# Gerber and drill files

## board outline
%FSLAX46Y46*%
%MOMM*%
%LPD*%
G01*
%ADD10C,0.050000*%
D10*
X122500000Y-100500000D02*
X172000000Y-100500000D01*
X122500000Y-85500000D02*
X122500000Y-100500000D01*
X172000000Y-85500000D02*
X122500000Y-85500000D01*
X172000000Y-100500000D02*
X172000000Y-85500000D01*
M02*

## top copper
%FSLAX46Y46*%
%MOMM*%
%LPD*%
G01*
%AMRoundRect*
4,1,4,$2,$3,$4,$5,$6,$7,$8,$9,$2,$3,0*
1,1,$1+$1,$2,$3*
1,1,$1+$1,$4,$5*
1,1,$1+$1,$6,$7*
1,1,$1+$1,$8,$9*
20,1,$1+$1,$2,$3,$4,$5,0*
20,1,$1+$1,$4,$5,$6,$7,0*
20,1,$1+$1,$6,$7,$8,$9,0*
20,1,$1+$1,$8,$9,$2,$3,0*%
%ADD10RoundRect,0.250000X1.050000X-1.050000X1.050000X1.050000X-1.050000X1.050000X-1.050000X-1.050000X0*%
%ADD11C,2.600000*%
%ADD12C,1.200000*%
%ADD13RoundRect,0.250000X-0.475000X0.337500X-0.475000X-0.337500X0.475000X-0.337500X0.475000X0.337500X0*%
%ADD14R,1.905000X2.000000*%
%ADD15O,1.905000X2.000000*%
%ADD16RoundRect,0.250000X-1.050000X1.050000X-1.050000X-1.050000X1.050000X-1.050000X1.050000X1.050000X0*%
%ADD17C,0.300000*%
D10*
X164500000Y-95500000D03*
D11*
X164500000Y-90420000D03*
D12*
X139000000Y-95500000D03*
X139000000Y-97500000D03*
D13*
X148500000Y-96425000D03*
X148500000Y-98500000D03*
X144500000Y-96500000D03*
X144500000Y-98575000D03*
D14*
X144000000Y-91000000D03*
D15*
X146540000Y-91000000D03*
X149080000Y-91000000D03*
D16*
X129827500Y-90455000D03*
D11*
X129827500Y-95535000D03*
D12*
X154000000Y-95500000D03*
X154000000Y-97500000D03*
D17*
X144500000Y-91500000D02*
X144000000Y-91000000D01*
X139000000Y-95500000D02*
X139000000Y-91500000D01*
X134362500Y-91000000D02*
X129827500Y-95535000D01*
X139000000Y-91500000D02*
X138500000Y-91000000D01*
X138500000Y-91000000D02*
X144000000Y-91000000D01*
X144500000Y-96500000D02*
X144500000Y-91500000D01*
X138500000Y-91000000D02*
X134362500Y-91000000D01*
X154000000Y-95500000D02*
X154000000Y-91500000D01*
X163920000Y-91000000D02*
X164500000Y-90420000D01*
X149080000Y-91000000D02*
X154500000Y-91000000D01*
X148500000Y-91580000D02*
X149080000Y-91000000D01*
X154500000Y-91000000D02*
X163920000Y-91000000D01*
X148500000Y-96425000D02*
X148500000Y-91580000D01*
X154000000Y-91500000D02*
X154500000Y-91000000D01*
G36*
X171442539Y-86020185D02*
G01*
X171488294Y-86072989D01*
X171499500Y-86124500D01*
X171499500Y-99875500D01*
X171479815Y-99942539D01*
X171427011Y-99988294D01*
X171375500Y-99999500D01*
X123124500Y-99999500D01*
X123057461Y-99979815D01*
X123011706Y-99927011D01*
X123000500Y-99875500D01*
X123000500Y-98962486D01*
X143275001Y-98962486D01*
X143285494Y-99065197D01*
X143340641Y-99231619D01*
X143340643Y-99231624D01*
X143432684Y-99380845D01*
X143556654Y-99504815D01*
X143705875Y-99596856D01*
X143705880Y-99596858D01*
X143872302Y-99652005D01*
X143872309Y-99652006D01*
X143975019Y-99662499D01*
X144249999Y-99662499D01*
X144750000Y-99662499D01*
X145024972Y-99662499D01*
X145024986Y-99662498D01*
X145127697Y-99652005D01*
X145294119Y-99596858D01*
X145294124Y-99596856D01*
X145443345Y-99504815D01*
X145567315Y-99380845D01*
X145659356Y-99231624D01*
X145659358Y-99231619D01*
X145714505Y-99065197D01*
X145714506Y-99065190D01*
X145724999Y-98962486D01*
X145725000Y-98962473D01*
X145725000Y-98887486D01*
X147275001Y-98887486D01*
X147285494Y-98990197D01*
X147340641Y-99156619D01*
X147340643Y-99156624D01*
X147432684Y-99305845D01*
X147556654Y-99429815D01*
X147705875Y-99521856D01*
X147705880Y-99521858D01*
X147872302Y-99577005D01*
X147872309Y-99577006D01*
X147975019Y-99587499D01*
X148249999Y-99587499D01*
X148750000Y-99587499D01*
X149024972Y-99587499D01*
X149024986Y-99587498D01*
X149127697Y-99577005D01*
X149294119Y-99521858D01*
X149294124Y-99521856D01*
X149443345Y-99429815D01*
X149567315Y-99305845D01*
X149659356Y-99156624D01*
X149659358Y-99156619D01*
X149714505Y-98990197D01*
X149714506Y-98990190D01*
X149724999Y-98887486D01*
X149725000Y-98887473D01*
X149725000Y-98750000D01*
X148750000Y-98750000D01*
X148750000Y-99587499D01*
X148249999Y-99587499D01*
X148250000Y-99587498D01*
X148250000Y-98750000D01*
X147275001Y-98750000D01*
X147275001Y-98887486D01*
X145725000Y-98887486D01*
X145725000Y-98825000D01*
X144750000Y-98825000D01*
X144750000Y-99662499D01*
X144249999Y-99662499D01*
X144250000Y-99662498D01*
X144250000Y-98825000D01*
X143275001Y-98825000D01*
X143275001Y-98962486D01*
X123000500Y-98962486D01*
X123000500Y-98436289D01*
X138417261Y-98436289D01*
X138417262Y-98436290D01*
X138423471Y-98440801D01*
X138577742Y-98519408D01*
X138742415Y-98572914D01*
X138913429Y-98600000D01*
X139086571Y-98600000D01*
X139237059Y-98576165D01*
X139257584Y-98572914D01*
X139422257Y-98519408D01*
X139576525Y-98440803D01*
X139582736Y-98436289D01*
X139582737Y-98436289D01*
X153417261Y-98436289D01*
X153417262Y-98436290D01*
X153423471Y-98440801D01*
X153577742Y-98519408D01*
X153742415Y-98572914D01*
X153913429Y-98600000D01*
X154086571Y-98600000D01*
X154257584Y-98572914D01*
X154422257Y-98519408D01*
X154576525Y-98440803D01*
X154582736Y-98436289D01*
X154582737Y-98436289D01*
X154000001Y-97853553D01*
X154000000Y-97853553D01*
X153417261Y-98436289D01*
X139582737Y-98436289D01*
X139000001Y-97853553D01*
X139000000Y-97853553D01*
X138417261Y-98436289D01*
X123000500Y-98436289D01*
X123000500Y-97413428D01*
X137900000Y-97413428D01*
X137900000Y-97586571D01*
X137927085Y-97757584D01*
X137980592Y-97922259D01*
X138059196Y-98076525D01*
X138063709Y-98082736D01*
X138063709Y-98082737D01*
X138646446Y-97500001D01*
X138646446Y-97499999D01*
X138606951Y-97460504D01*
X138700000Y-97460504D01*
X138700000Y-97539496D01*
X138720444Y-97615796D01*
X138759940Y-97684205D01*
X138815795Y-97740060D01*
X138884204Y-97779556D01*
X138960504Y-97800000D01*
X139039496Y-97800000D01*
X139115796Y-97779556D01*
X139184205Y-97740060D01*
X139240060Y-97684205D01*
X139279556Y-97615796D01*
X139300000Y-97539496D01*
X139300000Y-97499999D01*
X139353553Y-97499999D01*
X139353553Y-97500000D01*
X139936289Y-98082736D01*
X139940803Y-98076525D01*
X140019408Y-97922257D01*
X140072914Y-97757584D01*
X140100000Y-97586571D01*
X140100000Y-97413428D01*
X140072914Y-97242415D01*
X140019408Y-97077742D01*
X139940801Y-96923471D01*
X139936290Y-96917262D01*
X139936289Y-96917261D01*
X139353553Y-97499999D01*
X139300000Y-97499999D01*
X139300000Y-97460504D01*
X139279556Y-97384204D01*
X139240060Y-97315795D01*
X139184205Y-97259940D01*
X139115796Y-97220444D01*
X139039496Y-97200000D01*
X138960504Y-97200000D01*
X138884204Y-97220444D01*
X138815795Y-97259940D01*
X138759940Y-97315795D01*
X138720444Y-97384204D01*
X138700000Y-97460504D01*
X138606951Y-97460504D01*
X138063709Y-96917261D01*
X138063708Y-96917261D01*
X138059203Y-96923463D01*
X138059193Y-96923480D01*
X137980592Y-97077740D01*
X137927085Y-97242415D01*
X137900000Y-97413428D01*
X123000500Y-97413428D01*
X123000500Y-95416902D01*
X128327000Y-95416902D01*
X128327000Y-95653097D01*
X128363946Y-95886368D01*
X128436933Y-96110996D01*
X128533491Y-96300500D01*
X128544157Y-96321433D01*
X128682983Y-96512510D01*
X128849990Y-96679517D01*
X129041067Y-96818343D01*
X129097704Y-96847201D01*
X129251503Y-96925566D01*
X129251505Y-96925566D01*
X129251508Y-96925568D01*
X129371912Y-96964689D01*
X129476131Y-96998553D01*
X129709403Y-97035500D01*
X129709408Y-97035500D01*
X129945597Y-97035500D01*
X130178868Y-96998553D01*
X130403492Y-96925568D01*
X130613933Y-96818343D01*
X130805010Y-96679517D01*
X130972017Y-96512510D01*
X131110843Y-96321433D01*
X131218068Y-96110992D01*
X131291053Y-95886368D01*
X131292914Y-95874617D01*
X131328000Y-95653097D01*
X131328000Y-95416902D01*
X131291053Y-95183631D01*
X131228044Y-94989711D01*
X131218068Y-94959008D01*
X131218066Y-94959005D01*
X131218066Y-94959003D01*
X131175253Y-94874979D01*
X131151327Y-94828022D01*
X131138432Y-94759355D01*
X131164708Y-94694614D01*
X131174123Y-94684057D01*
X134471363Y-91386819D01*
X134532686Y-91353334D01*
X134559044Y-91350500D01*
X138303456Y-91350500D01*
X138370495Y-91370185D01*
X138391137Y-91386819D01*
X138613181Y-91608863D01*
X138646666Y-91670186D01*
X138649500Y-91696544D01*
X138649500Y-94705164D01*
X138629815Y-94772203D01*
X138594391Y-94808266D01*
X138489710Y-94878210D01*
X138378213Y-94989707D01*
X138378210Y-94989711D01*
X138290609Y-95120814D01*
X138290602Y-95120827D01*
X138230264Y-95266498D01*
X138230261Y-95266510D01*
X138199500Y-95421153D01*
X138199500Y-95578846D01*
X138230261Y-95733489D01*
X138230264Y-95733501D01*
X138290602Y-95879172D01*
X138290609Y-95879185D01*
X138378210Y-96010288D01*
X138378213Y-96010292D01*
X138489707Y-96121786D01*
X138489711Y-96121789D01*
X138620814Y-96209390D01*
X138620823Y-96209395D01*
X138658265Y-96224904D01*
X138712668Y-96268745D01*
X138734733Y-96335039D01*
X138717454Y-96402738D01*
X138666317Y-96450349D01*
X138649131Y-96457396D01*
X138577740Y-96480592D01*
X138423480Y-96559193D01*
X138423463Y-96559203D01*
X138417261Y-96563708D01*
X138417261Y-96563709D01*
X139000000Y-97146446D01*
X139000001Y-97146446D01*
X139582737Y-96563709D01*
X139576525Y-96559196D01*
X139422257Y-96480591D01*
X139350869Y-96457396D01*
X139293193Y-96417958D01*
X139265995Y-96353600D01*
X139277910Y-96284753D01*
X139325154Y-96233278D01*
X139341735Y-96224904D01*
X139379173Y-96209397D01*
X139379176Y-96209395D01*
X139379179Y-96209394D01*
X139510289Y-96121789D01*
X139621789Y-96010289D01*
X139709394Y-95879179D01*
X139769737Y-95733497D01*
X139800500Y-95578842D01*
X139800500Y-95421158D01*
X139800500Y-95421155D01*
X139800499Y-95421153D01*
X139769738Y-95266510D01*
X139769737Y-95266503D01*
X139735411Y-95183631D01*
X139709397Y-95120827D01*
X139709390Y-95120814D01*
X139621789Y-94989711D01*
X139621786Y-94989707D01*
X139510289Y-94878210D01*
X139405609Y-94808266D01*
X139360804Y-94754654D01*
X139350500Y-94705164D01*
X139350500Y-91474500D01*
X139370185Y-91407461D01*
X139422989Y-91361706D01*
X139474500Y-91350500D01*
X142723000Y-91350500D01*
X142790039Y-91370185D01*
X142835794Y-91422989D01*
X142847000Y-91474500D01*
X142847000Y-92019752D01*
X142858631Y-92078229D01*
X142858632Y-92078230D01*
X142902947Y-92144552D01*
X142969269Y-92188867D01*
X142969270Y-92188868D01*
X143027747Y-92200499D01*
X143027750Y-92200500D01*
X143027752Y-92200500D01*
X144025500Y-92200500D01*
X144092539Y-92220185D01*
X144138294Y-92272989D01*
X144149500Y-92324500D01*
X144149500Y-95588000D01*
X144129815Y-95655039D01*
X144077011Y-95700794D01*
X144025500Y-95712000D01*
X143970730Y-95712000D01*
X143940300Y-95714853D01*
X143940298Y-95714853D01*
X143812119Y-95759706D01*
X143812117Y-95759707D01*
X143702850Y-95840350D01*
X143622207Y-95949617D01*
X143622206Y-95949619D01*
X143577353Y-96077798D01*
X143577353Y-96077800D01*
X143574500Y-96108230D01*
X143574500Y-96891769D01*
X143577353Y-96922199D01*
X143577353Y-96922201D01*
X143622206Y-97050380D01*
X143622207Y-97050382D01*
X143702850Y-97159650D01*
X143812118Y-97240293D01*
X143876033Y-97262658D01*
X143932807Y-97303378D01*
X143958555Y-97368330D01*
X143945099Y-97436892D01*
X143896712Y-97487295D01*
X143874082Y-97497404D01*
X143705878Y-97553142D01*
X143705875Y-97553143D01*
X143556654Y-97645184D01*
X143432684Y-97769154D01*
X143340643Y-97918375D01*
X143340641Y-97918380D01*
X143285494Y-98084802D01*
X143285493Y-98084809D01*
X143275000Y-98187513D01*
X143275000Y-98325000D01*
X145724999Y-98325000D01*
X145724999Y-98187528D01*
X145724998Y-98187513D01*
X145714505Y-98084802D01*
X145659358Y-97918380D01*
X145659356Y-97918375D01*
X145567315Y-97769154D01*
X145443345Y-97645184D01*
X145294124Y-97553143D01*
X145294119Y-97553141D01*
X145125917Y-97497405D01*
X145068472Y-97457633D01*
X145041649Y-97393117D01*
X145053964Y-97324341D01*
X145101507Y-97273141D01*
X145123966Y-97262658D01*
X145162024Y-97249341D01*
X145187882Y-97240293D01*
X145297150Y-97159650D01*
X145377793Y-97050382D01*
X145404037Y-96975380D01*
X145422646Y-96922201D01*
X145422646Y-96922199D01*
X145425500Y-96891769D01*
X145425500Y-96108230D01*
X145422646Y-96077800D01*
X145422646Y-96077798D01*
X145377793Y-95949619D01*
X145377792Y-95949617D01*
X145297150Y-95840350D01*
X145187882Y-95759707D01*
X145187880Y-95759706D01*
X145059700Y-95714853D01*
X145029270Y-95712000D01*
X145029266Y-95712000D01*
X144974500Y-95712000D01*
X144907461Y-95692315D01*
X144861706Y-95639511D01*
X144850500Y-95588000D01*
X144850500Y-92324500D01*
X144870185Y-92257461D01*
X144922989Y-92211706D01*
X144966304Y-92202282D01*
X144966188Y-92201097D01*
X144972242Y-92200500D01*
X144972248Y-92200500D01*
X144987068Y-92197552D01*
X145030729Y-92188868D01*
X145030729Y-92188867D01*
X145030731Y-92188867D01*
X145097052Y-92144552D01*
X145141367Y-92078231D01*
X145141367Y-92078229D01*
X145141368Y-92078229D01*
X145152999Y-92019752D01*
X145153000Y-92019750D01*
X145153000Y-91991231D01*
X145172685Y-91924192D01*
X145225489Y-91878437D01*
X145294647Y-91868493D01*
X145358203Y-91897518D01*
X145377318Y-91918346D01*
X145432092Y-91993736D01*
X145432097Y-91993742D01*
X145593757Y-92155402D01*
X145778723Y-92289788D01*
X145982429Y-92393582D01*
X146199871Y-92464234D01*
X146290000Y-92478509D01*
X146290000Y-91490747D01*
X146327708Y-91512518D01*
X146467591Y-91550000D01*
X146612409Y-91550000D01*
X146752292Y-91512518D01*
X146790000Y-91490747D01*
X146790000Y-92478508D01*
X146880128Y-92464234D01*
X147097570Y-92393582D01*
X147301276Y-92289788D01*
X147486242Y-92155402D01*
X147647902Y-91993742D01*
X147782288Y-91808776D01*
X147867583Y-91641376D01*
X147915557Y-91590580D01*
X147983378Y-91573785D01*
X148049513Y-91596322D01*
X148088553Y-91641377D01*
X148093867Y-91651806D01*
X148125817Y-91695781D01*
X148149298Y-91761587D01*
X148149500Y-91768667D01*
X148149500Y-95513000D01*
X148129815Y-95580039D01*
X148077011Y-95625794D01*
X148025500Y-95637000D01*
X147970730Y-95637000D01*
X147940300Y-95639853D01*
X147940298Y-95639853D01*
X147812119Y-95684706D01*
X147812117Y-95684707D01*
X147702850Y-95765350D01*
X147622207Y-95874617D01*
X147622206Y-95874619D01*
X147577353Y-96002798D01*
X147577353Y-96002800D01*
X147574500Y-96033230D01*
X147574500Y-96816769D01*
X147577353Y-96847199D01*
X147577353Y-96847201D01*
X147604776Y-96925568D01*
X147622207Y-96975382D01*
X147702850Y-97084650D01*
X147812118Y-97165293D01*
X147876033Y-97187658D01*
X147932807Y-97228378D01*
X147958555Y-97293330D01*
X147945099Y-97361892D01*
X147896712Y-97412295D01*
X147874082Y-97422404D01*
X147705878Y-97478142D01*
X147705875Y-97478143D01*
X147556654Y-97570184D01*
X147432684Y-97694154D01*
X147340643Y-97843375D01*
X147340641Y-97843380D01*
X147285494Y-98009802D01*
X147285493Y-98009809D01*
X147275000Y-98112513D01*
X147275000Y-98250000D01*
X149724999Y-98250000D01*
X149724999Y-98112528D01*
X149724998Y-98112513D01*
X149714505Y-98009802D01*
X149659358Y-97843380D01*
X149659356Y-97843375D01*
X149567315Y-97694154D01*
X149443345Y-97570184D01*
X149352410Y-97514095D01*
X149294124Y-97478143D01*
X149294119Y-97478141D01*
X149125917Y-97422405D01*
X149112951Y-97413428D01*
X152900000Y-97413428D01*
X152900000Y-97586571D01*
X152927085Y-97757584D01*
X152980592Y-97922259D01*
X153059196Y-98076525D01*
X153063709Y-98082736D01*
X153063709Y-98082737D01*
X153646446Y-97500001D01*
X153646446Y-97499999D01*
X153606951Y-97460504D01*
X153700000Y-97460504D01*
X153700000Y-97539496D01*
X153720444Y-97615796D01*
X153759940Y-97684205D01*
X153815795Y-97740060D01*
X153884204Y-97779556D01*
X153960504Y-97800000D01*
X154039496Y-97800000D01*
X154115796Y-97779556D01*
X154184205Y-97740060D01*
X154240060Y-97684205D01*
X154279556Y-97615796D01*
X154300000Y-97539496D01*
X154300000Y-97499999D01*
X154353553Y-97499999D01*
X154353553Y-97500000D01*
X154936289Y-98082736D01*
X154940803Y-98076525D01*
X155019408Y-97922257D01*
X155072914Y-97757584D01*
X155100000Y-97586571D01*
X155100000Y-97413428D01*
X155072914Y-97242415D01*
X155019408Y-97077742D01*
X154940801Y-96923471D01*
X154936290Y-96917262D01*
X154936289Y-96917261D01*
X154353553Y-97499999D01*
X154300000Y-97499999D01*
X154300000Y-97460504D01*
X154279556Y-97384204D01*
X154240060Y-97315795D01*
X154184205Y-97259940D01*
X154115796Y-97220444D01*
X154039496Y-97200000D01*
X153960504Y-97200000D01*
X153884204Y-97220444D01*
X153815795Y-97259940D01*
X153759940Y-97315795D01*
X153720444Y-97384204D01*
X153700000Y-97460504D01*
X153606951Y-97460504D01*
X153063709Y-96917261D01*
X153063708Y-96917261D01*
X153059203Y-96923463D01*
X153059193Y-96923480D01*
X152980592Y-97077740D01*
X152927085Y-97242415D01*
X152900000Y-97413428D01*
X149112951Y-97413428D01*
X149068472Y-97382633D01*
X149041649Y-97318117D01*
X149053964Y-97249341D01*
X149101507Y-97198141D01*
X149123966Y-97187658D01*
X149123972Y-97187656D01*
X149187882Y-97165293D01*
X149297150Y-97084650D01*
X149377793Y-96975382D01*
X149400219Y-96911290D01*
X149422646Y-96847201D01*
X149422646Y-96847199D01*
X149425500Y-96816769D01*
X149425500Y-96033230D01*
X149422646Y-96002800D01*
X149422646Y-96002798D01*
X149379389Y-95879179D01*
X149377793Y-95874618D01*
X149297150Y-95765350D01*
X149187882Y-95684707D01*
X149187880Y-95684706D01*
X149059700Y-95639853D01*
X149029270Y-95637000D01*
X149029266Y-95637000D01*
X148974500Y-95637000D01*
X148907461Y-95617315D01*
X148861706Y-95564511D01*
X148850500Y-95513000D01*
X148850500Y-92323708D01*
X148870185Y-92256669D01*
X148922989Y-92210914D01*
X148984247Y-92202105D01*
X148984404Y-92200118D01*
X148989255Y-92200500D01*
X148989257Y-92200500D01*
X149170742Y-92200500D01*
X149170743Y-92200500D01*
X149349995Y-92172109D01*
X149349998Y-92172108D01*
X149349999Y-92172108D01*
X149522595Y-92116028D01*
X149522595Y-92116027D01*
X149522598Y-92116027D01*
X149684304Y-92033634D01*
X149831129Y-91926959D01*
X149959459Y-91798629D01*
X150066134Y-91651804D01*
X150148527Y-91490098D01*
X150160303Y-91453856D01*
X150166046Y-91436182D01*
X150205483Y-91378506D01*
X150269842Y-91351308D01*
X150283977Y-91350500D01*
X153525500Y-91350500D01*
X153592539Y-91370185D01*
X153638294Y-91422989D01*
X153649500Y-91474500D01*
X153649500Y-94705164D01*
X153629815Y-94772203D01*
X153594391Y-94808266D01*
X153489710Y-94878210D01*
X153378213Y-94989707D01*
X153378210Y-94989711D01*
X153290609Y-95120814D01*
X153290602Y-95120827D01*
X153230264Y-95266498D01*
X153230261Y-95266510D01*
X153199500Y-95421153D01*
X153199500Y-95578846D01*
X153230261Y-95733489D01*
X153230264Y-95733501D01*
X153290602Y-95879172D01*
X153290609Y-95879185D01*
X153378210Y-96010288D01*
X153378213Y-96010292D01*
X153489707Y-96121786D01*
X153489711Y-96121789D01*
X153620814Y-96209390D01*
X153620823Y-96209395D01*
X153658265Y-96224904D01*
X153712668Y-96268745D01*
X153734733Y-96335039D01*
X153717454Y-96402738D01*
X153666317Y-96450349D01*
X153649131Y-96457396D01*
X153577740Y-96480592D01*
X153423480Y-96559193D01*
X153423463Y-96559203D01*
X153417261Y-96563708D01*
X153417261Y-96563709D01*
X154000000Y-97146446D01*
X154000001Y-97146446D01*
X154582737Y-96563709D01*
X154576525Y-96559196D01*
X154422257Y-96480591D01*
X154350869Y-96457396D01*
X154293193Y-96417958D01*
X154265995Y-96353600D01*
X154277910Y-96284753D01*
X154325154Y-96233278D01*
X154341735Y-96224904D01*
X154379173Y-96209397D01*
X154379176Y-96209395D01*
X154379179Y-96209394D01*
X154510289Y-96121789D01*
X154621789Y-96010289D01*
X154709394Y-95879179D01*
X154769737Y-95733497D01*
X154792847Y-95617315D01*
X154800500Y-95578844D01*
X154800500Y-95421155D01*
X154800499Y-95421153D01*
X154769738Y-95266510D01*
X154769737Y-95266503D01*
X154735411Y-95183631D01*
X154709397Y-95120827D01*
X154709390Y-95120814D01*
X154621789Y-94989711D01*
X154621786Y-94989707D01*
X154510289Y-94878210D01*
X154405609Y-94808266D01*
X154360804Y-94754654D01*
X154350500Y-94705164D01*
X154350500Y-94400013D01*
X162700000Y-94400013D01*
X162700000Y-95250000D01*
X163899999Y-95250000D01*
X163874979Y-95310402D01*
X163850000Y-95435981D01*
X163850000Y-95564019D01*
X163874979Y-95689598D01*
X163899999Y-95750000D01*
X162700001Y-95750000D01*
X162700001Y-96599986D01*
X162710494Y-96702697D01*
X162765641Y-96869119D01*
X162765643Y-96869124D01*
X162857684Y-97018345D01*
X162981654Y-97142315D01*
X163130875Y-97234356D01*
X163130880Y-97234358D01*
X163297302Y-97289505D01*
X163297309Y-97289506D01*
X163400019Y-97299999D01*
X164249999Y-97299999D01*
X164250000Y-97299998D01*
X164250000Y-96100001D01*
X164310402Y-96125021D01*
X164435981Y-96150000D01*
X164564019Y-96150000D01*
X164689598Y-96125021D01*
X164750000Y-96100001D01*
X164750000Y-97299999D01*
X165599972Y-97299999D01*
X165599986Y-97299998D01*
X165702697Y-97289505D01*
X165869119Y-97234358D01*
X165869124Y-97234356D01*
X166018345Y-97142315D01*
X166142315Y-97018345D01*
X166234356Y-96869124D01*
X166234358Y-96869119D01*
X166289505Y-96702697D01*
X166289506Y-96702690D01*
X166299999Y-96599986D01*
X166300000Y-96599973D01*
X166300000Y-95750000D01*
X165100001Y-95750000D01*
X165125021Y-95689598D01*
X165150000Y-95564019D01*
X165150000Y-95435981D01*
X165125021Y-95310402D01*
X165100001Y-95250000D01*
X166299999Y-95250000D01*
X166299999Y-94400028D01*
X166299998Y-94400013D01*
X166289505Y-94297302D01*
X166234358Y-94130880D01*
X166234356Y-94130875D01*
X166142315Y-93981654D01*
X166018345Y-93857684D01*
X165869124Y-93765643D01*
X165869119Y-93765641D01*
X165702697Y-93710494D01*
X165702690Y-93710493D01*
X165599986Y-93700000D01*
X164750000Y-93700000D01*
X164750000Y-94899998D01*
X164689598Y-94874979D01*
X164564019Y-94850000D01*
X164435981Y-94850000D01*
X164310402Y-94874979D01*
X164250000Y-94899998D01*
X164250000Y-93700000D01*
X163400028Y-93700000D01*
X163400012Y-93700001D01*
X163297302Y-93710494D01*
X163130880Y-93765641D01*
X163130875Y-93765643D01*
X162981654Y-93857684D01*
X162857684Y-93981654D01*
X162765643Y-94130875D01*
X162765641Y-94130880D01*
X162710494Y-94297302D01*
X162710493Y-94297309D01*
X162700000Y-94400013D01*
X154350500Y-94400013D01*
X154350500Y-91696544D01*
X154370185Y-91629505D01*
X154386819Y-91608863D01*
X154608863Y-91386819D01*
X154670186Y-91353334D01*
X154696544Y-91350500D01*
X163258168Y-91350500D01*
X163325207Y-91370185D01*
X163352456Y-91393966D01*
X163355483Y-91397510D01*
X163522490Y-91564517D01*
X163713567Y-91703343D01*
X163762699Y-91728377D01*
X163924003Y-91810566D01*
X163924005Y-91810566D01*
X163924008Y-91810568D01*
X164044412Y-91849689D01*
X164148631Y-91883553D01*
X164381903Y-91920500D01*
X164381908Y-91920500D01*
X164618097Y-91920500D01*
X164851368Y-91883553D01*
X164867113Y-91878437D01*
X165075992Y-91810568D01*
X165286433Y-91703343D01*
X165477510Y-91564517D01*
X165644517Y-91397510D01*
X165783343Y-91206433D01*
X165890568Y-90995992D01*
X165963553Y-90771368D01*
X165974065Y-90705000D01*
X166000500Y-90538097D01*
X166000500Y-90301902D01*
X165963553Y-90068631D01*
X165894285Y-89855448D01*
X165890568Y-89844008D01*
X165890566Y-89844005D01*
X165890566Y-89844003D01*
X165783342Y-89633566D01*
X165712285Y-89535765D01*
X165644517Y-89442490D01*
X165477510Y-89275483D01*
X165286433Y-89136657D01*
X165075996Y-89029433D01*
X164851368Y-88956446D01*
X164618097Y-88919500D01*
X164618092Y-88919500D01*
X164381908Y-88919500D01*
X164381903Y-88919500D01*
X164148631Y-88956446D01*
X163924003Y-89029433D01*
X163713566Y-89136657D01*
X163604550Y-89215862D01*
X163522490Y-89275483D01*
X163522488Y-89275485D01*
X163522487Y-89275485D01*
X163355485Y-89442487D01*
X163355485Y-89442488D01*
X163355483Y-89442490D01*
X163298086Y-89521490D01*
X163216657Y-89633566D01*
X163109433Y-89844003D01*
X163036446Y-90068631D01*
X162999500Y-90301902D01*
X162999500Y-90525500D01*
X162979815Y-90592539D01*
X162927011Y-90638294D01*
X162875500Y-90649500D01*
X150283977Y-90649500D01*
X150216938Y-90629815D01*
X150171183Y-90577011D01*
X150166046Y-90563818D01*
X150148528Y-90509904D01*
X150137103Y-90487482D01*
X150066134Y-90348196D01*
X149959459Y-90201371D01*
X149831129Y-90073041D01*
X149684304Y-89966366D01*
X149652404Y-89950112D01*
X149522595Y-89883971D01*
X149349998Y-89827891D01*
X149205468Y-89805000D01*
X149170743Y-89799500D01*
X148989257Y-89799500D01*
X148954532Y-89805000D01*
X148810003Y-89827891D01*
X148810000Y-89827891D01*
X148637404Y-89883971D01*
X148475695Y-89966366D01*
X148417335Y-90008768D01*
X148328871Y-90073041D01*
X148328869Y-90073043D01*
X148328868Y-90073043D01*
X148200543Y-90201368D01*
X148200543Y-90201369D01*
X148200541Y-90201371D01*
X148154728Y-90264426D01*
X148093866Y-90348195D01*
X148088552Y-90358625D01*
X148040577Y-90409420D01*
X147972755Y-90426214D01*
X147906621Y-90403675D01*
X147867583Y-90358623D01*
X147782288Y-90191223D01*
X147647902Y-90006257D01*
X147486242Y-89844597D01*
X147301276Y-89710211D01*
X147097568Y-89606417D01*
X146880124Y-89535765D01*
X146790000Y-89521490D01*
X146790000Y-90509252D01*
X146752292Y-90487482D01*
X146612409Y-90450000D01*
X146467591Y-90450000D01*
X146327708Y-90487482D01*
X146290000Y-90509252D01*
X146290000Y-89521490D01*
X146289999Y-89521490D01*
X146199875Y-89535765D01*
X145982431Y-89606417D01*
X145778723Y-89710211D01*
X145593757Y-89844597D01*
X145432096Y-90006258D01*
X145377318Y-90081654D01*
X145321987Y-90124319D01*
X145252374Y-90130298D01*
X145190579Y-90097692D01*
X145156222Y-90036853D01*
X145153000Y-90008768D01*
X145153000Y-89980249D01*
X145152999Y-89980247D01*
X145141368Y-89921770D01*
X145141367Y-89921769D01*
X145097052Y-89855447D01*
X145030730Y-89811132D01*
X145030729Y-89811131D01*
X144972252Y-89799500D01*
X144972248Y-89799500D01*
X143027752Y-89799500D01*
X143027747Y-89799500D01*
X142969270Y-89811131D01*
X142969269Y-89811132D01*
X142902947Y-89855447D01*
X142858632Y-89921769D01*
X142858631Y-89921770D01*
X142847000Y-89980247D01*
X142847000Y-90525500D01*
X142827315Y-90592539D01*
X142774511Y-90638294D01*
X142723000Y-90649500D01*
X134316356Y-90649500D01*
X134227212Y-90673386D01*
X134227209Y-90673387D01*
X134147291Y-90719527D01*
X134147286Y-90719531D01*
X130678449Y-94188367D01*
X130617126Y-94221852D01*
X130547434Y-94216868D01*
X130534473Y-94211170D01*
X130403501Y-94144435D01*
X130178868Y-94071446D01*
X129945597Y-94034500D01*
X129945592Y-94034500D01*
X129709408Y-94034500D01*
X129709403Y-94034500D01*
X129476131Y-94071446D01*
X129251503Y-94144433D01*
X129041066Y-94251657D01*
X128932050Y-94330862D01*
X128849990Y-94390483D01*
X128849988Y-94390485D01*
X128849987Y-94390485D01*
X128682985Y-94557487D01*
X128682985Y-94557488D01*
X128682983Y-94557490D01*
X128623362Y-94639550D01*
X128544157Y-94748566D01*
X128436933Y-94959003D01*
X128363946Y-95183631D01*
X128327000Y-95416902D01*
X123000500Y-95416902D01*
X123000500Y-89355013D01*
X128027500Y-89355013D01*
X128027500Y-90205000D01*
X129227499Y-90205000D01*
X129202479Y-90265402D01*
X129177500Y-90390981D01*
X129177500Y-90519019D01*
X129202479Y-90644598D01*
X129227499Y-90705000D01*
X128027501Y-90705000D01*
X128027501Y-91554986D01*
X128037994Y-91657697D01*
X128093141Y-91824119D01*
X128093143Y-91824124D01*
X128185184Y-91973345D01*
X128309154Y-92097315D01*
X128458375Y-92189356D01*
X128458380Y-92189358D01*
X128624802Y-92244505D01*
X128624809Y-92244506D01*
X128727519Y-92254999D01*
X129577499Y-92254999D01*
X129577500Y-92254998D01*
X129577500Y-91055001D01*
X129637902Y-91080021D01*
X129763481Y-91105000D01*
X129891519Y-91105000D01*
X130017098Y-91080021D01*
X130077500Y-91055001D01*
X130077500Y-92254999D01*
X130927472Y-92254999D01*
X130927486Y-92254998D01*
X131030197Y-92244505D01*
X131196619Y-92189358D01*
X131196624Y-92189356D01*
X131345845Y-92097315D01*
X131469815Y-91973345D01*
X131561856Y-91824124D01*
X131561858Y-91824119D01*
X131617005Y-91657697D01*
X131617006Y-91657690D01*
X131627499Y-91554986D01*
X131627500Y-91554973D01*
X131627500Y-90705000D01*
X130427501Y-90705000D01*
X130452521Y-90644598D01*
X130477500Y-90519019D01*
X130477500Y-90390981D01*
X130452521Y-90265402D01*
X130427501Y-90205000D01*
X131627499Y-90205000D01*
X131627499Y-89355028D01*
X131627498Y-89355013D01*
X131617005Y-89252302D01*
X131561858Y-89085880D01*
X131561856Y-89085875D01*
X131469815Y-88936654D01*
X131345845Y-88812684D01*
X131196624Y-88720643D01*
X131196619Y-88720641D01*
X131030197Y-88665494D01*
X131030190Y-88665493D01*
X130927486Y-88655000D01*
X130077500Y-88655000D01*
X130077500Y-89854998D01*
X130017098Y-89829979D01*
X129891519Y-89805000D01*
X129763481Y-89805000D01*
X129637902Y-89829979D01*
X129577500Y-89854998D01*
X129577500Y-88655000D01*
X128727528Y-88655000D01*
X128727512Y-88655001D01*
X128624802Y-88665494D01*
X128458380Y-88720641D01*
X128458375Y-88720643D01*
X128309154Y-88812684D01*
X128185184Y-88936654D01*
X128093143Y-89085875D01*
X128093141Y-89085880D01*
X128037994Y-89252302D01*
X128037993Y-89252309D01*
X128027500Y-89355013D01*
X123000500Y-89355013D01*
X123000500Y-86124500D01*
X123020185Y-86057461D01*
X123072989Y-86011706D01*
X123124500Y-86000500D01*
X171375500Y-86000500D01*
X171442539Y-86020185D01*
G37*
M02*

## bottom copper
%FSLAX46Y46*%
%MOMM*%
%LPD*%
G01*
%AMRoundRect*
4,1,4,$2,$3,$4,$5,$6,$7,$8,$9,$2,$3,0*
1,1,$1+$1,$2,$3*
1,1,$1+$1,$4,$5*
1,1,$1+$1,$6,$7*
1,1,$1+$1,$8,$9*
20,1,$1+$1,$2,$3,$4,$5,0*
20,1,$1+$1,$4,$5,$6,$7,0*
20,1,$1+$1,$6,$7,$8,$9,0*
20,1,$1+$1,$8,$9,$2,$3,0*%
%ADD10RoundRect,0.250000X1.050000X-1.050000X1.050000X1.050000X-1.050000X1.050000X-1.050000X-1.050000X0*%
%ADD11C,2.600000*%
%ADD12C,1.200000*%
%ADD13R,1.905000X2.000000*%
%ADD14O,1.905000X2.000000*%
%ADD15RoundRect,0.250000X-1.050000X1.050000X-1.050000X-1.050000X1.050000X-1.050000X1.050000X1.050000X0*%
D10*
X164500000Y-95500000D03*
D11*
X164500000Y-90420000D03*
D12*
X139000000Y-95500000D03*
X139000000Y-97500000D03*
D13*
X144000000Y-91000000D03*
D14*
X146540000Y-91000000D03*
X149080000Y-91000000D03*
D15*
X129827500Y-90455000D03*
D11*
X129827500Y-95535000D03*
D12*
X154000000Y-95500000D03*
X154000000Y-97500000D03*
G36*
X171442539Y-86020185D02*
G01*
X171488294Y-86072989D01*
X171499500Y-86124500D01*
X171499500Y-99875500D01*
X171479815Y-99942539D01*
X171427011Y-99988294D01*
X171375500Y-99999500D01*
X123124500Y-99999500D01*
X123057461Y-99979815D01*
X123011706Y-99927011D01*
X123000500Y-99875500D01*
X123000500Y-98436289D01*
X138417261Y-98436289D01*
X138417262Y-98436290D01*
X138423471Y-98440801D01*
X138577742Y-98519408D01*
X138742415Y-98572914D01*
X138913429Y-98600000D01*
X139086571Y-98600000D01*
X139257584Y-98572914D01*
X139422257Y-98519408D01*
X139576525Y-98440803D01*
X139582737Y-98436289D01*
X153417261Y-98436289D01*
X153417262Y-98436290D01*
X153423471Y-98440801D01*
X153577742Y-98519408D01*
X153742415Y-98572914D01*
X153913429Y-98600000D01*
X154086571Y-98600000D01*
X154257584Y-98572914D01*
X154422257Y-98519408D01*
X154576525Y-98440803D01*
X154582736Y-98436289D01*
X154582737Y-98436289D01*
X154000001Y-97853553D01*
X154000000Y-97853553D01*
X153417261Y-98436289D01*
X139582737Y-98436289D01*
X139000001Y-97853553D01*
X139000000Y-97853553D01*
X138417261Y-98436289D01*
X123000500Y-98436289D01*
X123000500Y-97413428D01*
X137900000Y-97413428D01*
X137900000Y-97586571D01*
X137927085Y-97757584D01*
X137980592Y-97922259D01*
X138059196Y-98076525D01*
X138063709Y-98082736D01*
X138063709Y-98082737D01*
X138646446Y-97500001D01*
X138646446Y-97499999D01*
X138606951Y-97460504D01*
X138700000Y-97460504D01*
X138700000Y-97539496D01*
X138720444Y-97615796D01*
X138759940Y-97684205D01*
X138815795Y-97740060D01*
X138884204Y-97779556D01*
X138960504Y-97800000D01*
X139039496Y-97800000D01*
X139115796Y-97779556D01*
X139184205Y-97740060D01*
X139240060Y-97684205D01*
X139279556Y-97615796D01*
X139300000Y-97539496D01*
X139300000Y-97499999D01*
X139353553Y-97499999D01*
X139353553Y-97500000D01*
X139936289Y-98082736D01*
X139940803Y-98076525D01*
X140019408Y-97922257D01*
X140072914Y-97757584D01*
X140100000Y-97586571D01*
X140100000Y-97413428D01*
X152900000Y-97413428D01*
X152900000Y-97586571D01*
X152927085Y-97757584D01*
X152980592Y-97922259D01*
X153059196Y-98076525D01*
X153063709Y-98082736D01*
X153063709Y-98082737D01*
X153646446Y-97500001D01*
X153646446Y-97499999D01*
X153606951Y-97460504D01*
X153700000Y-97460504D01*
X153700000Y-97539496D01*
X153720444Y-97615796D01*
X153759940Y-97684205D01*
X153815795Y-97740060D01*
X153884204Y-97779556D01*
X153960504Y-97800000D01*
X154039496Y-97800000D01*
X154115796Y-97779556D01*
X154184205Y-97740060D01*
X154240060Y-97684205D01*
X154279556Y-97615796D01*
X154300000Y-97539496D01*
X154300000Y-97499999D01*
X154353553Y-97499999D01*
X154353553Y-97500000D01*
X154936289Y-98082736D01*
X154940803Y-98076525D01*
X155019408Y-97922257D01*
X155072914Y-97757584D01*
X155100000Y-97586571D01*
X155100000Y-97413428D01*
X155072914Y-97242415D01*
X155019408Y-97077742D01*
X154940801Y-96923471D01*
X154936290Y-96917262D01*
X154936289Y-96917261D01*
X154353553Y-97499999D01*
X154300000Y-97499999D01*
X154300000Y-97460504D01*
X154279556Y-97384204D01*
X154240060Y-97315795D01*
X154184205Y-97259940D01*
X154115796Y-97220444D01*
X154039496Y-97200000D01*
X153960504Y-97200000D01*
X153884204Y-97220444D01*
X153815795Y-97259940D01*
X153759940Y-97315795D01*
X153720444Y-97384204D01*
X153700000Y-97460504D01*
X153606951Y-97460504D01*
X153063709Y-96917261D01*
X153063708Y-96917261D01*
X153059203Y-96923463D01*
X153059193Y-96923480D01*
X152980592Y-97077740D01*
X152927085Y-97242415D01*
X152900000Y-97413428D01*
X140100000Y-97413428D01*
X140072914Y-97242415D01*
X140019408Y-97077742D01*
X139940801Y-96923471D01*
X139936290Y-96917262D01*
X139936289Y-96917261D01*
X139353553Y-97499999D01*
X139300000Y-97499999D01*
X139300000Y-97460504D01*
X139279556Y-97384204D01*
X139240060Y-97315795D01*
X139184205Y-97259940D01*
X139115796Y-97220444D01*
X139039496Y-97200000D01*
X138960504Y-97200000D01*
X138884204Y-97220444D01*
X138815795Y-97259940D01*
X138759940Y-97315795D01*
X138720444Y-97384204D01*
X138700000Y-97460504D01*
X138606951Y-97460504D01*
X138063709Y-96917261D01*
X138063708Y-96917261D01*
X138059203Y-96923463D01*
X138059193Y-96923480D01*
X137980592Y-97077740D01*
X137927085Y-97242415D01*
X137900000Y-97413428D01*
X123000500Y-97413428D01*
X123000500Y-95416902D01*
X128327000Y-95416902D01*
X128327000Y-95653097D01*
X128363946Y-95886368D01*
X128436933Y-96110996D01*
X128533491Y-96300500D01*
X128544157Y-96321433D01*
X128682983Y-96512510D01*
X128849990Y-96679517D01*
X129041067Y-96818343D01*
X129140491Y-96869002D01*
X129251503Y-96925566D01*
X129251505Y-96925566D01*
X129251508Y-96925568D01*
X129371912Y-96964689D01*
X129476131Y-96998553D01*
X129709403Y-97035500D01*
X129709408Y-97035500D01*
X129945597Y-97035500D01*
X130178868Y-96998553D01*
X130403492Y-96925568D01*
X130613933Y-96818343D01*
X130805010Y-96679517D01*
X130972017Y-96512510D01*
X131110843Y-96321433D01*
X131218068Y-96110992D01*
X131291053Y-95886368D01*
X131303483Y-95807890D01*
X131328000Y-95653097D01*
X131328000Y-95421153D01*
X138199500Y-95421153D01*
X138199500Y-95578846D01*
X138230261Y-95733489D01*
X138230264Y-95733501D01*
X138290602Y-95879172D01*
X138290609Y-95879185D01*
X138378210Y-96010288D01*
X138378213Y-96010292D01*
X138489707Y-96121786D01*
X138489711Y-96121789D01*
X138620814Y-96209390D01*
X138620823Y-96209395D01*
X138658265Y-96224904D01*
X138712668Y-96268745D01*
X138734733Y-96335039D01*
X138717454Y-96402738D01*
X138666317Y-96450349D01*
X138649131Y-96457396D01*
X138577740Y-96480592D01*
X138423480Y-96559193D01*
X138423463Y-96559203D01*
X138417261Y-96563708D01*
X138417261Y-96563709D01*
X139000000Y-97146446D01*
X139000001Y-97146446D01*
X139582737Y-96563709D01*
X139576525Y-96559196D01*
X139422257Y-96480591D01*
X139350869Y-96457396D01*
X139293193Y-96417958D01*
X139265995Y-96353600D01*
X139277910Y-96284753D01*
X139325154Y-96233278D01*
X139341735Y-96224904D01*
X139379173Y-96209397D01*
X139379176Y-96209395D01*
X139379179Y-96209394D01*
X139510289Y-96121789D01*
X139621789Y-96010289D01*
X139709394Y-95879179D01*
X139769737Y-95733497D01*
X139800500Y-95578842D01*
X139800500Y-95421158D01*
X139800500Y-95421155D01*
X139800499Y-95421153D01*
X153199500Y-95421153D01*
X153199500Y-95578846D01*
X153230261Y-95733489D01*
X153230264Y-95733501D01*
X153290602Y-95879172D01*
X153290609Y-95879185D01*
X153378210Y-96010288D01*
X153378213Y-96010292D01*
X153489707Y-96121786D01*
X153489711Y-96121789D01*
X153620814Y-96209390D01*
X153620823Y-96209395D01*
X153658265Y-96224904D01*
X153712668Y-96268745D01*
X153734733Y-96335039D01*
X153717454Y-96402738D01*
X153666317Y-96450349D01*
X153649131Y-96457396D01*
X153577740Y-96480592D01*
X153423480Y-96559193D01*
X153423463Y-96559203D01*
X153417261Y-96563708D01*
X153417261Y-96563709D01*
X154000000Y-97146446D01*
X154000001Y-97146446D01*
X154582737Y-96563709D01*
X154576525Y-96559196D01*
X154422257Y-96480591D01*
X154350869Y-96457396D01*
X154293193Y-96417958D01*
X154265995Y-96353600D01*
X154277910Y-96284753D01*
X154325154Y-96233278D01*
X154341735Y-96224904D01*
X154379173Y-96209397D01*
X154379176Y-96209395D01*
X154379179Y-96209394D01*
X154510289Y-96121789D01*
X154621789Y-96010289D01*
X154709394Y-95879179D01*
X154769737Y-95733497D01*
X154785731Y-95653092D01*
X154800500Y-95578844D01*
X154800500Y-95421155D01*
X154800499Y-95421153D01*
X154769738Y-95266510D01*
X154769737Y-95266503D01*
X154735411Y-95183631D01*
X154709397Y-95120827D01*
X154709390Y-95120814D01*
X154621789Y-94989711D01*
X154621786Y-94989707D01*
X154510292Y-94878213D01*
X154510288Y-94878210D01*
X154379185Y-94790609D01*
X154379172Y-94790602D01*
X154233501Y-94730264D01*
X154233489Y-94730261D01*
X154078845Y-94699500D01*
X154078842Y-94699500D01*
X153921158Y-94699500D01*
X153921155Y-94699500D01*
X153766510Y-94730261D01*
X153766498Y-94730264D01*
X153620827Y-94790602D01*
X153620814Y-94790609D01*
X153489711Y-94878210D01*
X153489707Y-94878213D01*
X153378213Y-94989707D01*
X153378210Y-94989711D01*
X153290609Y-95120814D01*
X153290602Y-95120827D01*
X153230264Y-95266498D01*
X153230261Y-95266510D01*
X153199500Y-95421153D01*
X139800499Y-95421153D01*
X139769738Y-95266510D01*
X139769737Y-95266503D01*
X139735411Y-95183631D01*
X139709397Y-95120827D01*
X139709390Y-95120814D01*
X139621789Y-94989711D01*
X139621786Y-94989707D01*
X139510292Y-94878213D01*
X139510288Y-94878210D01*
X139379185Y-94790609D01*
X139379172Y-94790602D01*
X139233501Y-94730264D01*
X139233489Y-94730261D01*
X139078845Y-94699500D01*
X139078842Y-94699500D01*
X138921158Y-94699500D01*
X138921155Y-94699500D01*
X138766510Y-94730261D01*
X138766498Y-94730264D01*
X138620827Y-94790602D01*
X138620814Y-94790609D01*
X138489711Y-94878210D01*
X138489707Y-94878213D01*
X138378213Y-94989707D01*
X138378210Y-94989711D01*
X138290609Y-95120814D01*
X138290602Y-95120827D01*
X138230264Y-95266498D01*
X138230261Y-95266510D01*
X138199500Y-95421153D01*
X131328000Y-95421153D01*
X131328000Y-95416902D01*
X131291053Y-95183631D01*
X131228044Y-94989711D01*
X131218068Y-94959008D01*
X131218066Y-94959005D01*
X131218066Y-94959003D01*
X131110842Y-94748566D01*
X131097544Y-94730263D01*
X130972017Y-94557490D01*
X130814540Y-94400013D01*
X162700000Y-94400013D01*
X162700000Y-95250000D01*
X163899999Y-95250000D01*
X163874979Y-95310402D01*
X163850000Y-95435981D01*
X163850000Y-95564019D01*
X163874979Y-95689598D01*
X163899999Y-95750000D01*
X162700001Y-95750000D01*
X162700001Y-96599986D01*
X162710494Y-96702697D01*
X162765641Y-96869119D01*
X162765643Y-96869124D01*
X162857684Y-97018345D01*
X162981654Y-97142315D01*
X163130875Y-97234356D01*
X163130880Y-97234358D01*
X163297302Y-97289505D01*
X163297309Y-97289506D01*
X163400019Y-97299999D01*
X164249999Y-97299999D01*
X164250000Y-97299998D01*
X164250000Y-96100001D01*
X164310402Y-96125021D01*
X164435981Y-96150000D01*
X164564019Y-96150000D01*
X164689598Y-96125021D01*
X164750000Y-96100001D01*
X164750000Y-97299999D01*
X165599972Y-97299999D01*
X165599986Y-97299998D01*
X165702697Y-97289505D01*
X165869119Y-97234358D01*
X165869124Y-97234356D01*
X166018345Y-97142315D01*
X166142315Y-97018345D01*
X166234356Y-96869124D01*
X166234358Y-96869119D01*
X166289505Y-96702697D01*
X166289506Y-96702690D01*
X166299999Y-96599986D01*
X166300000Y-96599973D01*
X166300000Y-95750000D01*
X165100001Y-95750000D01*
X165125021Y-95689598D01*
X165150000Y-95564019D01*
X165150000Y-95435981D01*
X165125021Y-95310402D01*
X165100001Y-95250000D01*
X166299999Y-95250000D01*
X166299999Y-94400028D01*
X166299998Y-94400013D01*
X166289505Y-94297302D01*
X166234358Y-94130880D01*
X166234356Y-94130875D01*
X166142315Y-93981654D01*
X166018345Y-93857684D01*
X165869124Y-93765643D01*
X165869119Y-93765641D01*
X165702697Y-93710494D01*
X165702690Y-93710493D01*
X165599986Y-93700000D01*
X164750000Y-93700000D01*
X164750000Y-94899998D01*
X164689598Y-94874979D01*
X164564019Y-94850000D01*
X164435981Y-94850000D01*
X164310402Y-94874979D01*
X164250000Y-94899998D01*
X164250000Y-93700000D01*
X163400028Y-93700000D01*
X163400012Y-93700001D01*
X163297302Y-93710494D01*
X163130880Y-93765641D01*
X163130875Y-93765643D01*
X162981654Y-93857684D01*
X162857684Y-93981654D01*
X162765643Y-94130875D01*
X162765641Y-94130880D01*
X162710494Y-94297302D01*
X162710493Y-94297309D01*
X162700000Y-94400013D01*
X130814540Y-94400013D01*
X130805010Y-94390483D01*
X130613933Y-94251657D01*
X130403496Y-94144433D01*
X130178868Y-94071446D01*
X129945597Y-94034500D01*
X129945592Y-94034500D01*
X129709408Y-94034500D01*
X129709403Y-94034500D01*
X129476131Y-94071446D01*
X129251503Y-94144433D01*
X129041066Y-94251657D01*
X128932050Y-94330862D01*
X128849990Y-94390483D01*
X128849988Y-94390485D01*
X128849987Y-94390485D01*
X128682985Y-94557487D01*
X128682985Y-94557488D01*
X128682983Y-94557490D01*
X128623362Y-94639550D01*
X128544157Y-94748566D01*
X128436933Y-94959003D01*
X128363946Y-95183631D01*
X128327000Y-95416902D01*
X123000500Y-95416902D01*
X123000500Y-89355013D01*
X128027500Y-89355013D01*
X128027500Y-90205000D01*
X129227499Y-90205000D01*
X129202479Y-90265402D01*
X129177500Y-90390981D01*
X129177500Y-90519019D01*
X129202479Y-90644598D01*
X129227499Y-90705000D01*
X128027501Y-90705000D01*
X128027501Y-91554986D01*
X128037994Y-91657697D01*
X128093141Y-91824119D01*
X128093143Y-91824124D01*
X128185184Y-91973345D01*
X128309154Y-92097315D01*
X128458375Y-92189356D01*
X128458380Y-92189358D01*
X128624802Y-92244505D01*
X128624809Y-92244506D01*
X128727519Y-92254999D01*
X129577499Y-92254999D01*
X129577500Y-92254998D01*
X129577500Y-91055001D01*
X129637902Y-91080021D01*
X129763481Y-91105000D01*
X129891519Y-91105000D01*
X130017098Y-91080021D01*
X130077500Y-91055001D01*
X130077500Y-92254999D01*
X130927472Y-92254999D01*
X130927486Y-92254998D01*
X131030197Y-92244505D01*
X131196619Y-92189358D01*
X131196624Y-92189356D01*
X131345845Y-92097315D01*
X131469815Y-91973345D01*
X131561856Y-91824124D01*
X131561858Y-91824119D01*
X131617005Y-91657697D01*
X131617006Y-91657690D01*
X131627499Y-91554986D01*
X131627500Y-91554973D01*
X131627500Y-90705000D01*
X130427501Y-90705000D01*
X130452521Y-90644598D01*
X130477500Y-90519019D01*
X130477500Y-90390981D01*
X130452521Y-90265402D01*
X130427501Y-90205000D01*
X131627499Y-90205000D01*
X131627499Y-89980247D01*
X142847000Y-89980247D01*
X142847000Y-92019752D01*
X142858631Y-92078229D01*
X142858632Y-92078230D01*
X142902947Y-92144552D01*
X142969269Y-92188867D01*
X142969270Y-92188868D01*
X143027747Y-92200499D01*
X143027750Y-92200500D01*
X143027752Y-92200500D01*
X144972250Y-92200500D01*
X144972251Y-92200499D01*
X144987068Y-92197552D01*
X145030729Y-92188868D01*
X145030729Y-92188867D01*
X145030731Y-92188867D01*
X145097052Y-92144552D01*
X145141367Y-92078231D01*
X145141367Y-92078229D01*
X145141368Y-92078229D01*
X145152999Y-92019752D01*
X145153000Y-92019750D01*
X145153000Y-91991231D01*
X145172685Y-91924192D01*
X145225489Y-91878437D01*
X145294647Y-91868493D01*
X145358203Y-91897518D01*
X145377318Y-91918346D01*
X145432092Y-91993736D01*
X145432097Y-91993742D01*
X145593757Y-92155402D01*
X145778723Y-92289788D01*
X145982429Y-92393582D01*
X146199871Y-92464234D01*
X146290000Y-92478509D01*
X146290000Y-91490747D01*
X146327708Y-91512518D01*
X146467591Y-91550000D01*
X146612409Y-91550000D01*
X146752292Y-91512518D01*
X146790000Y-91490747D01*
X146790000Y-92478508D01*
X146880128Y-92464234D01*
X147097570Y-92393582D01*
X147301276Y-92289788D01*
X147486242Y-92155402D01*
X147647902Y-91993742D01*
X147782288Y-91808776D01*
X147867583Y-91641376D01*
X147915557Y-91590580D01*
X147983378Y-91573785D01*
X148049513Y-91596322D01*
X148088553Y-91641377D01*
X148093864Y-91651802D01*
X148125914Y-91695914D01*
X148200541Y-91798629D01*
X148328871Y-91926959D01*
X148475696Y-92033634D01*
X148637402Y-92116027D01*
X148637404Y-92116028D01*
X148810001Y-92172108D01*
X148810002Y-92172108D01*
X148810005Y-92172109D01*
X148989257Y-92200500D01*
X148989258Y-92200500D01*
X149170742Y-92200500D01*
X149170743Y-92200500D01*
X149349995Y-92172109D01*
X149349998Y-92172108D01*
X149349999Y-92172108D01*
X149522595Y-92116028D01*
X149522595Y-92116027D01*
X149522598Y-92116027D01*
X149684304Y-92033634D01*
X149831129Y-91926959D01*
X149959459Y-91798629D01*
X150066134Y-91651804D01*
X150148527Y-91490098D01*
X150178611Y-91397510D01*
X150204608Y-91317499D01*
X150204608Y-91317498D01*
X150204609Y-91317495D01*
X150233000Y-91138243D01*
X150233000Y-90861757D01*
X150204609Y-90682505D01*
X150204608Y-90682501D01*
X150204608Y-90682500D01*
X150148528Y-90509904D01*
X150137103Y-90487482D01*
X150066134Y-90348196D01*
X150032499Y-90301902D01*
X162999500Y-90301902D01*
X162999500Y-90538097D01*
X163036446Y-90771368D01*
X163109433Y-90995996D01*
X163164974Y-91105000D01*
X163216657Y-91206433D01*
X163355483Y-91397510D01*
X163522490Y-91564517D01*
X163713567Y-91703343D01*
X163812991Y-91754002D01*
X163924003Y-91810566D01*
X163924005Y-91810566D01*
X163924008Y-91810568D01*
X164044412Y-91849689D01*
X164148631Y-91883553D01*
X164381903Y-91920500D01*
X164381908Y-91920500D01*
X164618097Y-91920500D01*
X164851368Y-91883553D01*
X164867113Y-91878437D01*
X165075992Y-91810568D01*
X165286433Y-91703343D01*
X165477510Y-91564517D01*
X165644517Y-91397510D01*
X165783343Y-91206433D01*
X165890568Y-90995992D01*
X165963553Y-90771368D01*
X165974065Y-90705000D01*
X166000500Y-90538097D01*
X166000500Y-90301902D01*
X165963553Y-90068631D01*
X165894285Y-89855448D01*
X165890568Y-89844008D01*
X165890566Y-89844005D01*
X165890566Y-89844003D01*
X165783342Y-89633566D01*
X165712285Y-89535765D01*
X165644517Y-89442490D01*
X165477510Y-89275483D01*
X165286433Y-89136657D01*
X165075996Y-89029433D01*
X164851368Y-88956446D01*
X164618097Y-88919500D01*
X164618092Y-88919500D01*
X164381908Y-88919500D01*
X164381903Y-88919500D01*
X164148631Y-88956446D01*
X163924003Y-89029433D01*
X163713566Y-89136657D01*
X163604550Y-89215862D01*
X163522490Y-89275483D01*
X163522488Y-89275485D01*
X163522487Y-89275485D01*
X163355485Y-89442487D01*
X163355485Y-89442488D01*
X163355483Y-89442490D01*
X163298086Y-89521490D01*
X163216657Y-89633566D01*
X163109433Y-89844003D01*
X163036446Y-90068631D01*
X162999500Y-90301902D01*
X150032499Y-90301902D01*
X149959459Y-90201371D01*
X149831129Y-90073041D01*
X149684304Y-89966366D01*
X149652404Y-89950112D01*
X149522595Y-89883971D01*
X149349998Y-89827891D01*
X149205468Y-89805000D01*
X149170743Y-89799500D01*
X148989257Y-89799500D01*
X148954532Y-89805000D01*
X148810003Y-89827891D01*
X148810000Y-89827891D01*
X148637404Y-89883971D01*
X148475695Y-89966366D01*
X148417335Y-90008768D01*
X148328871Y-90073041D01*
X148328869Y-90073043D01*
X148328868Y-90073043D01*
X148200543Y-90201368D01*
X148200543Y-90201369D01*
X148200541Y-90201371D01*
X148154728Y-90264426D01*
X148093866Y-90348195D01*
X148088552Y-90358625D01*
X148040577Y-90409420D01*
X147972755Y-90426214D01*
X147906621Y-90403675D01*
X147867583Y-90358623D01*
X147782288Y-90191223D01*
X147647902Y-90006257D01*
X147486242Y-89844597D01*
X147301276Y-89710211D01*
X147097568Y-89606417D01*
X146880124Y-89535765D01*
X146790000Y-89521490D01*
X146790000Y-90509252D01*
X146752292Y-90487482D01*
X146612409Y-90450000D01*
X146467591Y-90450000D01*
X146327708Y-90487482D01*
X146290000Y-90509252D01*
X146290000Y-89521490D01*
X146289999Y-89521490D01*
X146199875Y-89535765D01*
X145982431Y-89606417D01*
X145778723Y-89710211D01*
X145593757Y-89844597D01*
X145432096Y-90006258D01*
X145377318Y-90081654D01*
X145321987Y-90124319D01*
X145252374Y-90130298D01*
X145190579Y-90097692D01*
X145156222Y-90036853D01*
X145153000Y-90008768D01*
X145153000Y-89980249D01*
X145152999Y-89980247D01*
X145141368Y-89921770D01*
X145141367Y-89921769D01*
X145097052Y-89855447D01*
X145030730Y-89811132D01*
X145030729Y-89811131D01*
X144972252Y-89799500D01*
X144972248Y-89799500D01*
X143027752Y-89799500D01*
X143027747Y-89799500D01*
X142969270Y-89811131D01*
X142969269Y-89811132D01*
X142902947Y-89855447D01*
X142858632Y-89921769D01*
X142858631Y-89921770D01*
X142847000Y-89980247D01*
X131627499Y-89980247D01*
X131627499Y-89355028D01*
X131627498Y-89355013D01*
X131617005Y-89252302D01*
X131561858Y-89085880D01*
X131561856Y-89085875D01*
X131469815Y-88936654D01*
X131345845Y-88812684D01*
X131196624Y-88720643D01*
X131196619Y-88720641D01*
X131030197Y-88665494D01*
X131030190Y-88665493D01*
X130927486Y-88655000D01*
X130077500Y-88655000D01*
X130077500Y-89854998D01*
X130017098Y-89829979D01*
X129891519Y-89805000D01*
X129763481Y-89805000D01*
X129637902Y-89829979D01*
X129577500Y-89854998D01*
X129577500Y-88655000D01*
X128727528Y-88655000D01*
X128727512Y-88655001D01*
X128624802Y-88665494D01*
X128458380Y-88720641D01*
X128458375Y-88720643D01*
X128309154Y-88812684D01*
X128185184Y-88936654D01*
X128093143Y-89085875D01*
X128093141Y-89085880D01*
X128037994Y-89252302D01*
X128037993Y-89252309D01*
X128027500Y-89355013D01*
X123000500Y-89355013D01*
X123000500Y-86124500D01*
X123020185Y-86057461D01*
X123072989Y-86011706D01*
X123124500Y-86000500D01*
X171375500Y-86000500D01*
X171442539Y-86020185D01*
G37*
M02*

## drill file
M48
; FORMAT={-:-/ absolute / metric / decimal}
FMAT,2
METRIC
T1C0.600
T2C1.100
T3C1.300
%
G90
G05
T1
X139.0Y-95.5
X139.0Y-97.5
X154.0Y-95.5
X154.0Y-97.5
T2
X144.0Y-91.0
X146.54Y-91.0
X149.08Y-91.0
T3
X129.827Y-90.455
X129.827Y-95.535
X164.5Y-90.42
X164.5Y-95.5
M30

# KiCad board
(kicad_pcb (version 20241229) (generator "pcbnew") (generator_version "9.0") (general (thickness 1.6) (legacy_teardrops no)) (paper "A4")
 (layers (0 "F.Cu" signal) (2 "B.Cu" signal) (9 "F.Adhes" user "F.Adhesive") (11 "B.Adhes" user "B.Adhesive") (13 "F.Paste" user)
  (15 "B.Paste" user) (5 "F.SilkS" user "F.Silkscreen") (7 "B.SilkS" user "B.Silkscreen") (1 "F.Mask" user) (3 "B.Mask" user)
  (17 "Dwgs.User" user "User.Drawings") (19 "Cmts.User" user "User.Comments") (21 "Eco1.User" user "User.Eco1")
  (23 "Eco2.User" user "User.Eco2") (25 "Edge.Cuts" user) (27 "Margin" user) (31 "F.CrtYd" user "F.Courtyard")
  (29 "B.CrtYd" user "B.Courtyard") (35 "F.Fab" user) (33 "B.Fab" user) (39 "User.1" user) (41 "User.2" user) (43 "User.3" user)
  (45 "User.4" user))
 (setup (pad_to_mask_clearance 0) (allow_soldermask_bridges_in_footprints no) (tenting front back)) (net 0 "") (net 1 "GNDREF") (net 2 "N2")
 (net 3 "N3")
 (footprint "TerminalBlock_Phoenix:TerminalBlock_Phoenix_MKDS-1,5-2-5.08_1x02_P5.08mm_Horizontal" (layer "F.Cu") (at 164.5 95.5 90)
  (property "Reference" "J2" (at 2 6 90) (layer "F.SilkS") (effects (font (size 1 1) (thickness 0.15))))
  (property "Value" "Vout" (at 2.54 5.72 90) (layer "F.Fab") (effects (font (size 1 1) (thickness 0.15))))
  (pad "1" thru_hole roundrect (at 0 0 90) (size 2.6 2.6) (drill 1.3) (layers "*.Cu" "*.Mask") (remove_unused_layers no)
   (roundrect_rratio 0.096154) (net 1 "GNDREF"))
  (pad "2" thru_hole circle (at 5.08 0 90) (size 2.6 2.6) (drill 1.3) (layers "*.Cu" "*.Mask") (remove_unused_layers no) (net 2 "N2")))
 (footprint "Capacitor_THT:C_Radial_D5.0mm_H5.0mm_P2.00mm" (layer "F.Cu") (at 139 95.5 -90)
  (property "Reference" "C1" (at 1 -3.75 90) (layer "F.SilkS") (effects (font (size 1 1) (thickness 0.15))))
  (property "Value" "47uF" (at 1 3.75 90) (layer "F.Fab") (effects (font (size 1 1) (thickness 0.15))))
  (pad "1" thru_hole circle (at 0 0 270) (size 1.2 1.2) (drill 0.6) (layers "*.Cu" "*.Mask") (remove_unused_layers no) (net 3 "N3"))
  (pad "2" thru_hole circle (at 2 0 270) (size 1.2 1.2) (drill 0.6) (layers "*.Cu" "*.Mask") (remove_unused_layers no) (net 1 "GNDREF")))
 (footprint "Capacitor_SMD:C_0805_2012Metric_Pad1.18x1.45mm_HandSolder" (layer "F.Cu") (at 148.5 97.4625 -90)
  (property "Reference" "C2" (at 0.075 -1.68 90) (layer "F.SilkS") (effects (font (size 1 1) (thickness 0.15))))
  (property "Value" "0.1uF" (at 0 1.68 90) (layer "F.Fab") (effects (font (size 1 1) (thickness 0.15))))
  (pad "1" smd roundrect (at -1.0375 0 270) (size 1.175 1.45) (layers "F.Cu" "F.Mask" "F.Paste") (roundrect_rratio 0.212766) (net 2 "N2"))
  (pad "2" smd roundrect (at 1.0375 0 270) (size 1.175 1.45) (layers "F.Cu" "F.Mask" "F.Paste") (roundrect_rratio 0.212766) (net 1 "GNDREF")))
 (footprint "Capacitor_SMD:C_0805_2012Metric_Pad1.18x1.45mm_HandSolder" (layer "F.Cu") (at 144.5 97.5375 -90)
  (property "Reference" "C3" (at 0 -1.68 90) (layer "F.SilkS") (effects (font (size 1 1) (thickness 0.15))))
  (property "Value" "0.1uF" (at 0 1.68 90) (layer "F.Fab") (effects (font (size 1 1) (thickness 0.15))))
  (pad "1" smd roundrect (at -1.0375 0 270) (size 1.175 1.45) (layers "F.Cu" "F.Mask" "F.Paste") (roundrect_rratio 0.212766) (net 3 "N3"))
  (pad "2" smd roundrect (at 1.0375 0 270) (size 1.175 1.45) (layers "F.Cu" "F.Mask" "F.Paste") (roundrect_rratio 0.212766) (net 1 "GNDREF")))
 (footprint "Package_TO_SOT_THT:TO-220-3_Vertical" (layer "F.Cu") (at 144 91)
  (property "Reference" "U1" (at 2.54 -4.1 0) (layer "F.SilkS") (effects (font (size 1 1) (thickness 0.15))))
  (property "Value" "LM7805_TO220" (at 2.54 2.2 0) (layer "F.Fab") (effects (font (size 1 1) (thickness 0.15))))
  (pad "1" thru_hole rect (at 0 0) (size 1.905 2) (drill 1.1) (layers "*.Cu" "*.Mask") (remove_unused_layers no) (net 3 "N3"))
  (pad "2" thru_hole oval (at 2.54 0) (size 1.905 2) (drill 1.1) (layers "*.Cu" "*.Mask") (remove_unused_layers no) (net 1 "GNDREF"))
  (pad "3" thru_hole oval (at 5.08 0) (size 1.905 2) (drill 1.1) (layers "*.Cu" "*.Mask") (remove_unused_layers no) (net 2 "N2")))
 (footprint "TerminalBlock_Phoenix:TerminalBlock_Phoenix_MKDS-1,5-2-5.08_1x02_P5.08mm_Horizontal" (layer "F.Cu") (at 129.8275 90.455 -90)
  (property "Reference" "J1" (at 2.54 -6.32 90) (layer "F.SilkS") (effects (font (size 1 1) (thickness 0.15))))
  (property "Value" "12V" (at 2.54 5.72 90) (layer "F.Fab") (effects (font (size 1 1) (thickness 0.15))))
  (pad "1" thru_hole roundrect (at 0 0 270) (size 2.6 2.6) (drill 1.3) (layers "*.Cu" "*.Mask") (remove_unused_layers no)
   (roundrect_rratio 0.096154) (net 1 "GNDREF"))
  (pad "2" thru_hole circle (at 5.08 0 270) (size 2.6 2.6) (drill 1.3) (layers "*.Cu" "*.Mask") (remove_unused_layers no) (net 3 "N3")))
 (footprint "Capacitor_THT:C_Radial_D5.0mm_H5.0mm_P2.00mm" (layer "F.Cu") (at 154 95.5 -90)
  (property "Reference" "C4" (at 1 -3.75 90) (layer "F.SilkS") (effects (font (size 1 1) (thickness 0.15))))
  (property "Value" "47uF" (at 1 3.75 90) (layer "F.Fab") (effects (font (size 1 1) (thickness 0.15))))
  (pad "1" thru_hole circle (at 0 0 270) (size 1.2 1.2) (drill 0.6) (layers "*.Cu" "*.Mask") (remove_unused_layers no) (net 2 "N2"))
  (pad "2" thru_hole circle (at 2 0 270) (size 1.2 1.2) (drill 0.6) (layers "*.Cu" "*.Mask") (remove_unused_layers no) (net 1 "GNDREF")))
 (gr_line (start 122.5 100.5) (end 172 100.5) (stroke (width 0.05) (type default)) (layer "Edge.Cuts"))
 (gr_line (start 122.5 85.5) (end 122.5 100.5) (stroke (width 0.05) (type default)) (layer "Edge.Cuts"))
 (gr_line (start 172 85.5) (end 122.5 85.5) (stroke (width 0.05) (type default)) (layer "Edge.Cuts"))
 (gr_line (start 172 100.5) (end 172 85.5) (stroke (width 0.05) (type default)) (layer "Edge.Cuts"))
 (segment (start 144.5 91.5) (end 144 91) (width 0.3) (layer "F.Cu") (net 3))
 (segment (start 139 95.5) (end 139 91.5) (width 0.3) (layer "F.Cu") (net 3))
 (segment (start 134.3625 91) (end 129.8275 95.535) (width 0.3) (layer "F.Cu") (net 3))
 (segment (start 139 91.5) (end 138.5 91) (width 0.3) (layer "F.Cu") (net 3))
 (segment (start 138.5 91) (end 144 91) (width 0.3) (layer "F.Cu") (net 3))
 (segment (start 144.5 96.5) (end 144.5 91.5) (width 0.3) (layer "F.Cu") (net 3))
 (segment (start 138.5 91) (end 134.3625 91) (width 0.3) (layer "F.Cu") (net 3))
 (segment (start 154 95.5) (end 154 91.5) (width 0.3) (layer "F.Cu") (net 2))
 (segment (start 163.92 91) (end 164.5 90.42) (width 0.3) (layer "F.Cu") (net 2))
 (segment (start 149.08 91) (end 154.5 91) (width 0.3) (layer "F.Cu") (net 2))
 (segment (start 148.5 91.58) (end 149.08 91) (width 0.3) (layer "F.Cu") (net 2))
 (segment (start 154.5 91) (end 163.92 91) (width 0.3) (layer "F.Cu") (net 2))
 (segment (start 148.5 96.425) (end 148.5 91.58) (width 0.3) (layer "F.Cu") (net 2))
 (segment (start 154 91.5) (end 154.5 91) (width 0.3) (layer "F.Cu") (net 2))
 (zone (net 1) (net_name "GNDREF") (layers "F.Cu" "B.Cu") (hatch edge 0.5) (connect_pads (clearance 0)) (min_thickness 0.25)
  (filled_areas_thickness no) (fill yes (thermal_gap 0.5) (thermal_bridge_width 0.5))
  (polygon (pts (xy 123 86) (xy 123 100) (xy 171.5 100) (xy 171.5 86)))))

